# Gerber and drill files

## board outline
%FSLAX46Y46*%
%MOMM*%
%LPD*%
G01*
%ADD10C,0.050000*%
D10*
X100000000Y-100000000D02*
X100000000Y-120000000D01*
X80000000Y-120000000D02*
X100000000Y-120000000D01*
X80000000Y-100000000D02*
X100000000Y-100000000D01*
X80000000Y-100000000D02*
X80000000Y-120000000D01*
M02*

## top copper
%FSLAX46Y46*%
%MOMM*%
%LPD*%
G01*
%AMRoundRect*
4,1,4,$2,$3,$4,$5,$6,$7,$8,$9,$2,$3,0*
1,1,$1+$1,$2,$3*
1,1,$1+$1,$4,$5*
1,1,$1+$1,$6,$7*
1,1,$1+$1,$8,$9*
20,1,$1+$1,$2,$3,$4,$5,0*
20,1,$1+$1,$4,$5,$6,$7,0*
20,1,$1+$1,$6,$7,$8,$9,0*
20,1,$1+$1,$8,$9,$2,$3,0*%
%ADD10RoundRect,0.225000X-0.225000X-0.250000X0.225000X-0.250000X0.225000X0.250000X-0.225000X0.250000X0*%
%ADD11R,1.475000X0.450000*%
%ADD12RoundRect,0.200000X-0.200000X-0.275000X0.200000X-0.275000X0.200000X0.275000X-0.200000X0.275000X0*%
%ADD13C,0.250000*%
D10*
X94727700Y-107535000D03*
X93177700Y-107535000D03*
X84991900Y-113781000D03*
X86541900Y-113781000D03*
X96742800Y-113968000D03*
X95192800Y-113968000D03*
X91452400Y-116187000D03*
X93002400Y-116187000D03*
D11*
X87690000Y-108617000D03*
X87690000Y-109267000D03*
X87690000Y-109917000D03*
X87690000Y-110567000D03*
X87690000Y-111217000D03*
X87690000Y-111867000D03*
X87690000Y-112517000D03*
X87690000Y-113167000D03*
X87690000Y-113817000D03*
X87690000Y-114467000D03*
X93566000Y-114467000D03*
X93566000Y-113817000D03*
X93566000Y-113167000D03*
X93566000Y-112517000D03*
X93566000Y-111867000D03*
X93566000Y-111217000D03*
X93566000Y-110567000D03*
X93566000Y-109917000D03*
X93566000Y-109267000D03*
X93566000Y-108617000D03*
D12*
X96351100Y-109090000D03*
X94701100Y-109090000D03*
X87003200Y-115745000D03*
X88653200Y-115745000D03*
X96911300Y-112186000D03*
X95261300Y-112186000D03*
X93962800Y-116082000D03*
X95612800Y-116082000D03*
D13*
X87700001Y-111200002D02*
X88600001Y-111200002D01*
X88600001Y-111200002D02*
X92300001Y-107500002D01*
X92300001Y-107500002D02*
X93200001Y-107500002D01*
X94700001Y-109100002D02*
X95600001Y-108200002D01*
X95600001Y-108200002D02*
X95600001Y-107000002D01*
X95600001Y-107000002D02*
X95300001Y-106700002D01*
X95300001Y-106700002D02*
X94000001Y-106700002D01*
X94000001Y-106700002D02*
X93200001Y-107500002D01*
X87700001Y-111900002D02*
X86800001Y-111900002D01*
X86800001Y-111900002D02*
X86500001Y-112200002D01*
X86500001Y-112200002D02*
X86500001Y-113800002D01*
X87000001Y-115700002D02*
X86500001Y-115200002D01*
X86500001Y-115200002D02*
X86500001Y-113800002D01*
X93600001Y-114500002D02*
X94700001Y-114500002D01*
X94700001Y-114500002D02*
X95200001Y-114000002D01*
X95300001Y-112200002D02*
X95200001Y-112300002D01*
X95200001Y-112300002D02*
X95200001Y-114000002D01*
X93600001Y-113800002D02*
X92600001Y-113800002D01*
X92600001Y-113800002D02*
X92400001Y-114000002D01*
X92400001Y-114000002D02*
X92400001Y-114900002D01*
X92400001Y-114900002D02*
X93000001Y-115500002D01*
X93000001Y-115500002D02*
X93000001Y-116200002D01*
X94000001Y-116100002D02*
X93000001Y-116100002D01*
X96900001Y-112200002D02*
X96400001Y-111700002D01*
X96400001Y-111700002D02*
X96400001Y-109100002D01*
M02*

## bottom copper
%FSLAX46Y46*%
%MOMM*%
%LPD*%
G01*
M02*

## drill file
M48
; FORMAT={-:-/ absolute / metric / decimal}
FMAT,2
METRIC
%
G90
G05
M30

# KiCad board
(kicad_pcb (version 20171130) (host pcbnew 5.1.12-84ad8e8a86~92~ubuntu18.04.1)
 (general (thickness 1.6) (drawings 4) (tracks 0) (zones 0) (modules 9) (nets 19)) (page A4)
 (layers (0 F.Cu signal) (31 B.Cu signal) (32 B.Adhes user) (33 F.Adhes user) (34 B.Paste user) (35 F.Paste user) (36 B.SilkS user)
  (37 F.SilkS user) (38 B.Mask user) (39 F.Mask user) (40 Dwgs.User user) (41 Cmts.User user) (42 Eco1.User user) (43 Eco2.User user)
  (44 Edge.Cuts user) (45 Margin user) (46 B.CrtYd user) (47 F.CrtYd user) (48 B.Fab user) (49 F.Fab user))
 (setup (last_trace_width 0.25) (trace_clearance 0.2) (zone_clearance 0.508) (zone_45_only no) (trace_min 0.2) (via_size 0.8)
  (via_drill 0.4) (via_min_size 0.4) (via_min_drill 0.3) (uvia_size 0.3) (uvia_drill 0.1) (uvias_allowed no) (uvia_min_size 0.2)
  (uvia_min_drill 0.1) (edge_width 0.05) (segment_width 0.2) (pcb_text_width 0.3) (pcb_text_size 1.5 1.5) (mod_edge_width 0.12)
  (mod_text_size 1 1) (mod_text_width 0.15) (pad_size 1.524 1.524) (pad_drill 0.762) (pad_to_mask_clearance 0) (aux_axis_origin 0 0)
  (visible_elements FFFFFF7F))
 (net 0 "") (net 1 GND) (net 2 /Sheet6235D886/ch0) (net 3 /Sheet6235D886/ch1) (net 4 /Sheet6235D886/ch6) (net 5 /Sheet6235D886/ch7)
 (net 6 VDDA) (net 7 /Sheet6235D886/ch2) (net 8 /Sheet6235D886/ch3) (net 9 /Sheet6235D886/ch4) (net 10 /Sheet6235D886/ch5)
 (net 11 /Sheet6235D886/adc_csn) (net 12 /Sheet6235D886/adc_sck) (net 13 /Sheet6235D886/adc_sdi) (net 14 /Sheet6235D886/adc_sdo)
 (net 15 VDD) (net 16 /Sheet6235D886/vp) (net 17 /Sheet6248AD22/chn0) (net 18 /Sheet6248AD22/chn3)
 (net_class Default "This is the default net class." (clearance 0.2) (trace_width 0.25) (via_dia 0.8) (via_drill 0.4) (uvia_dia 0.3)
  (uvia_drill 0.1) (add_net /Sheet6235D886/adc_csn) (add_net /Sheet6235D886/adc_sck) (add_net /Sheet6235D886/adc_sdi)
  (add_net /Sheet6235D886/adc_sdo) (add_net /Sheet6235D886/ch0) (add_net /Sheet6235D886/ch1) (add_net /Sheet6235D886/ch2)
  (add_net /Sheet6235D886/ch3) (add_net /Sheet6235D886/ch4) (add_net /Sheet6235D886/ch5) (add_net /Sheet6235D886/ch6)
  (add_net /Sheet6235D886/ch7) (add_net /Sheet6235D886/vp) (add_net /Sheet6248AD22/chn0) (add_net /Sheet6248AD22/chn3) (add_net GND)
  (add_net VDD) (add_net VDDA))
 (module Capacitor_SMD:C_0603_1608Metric (layer F.Cu) (at 93.952700 107.535000)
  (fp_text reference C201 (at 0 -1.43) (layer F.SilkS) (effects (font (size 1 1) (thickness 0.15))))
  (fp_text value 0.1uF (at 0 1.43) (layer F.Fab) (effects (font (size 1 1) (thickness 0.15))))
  (pad 2 smd roundrect (at 0.775 0) (size 0.9 0.95) (layers F.Cu F.Mask F.Paste) (roundrect_rratio 0.25) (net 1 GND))
  (pad 1 smd roundrect (at -0.775 0) (size 0.9 0.95) (layers F.Cu F.Mask F.Paste) (roundrect_rratio 0.25) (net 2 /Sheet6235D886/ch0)))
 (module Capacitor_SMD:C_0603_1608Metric (layer F.Cu) (at 85.766900 113.781000)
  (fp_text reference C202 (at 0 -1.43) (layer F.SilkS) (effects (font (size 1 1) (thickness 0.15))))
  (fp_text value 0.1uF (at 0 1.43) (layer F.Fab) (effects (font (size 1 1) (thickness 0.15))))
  (pad 1 smd roundrect (at -0.775 0) (size 0.9 0.95) (layers F.Cu F.Mask F.Paste) (roundrect_rratio 0.25) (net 1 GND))
  (pad 2 smd roundrect (at 0.775 0) (size 0.9 0.95) (layers F.Cu F.Mask F.Paste) (roundrect_rratio 0.25) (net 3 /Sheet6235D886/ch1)))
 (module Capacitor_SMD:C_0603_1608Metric (layer F.Cu) (at 95.967800 113.968000)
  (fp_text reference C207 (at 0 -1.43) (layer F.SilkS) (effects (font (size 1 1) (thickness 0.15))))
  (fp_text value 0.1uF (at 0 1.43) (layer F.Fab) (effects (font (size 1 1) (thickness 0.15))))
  (pad 2 smd roundrect (at 0.775 0) (size 0.9 0.95) (layers F.Cu F.Mask F.Paste) (roundrect_rratio 0.25) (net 1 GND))
  (pad 1 smd roundrect (at -0.775 0) (size 0.9 0.95) (layers F.Cu F.Mask F.Paste) (roundrect_rratio 0.25) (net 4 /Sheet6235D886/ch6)))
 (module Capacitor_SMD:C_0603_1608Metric (layer F.Cu) (at 92.227400 116.187000)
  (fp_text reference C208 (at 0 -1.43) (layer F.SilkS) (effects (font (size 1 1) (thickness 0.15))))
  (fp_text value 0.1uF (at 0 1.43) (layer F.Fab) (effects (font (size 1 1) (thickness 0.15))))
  (pad 1 smd roundrect (at -0.775 0) (size 0.9 0.95) (layers F.Cu F.Mask F.Paste) (roundrect_rratio 0.25) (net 1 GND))
  (pad 2 smd roundrect (at 0.775 0) (size 0.9 0.95) (layers F.Cu F.Mask F.Paste) (roundrect_rratio 0.25) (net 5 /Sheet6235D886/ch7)))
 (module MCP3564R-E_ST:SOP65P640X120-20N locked (layer F.Cu) (at 90.628000 111.542000)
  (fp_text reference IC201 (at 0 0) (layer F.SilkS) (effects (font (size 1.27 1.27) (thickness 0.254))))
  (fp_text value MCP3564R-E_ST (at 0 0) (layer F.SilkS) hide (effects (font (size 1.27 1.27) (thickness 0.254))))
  (pad 1 smd rect (at -2.938 -2.925 90.000000) (size 0.45 1.475) (layers F.Cu F.Mask F.Paste) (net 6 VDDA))
  (pad 2 smd rect (at -2.938 -2.275 90.000000) (size 0.45 1.475) (layers F.Cu F.Mask F.Paste) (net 1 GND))
  (pad 3 smd rect (at -2.938 -1.625 90.000000) (size 0.45 1.475) (layers F.Cu F.Mask F.Paste) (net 1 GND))
  (pad 4 smd rect (at -2.938 -0.975 90.000000) (size 0.45 1.475) (layers F.Cu F.Mask F.Paste))
  (pad 5 smd rect (at -2.938 -0.325 90.000000) (size 0.45 1.475) (layers F.Cu F.Mask F.Paste) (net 2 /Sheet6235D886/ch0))
  (pad 6 smd rect (at -2.938 0.325 90.000000) (size 0.45 1.475) (layers F.Cu F.Mask F.Paste) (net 3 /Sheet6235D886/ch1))
  (pad 7 smd rect (at -2.938 0.975 90.000000) (size 0.45 1.475) (layers F.Cu F.Mask F.Paste) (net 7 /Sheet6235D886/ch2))
  (pad 8 smd rect (at -2.938 1.625 90.000000) (size 0.45 1.475) (layers F.Cu F.Mask F.Paste) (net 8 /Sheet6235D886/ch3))
  (pad 9 smd rect (at -2.938 2.275 90.000000) (size 0.45 1.475) (layers F.Cu F.Mask F.Paste) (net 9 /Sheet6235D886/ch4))
  (pad 10 smd rect (at -2.938 2.925 90.000000) (size 0.45 1.475) (layers F.Cu F.Mask F.Paste) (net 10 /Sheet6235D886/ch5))
  (pad 11 smd rect (at 2.938 2.925 90.000000) (size 0.45 1.475) (layers F.Cu F.Mask F.Paste) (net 4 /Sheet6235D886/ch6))
  (pad 12 smd rect (at 2.938 2.275 90.000000) (size 0.45 1.475) (layers F.Cu F.Mask F.Paste) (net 5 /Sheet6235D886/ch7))
  (pad 13 smd rect (at 2.938 1.625 90.000000) (size 0.45 1.475) (layers F.Cu F.Mask F.Paste) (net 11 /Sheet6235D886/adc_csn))
  (pad 14 smd rect (at 2.938 0.975 90.000000) (size 0.45 1.475) (layers F.Cu F.Mask F.Paste) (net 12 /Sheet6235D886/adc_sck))
  (pad 15 smd rect (at 2.938 0.325 90.000000) (size 0.45 1.475) (layers F.Cu F.Mask F.Paste) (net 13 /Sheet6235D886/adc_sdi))
  (pad 16 smd rect (at 2.938 -0.325 90.000000) (size 0.45 1.475) (layers F.Cu F.Mask F.Paste) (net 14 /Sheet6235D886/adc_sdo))
  (pad 17 smd rect (at 2.938 -0.975 90.000000) (size 0.45 1.475) (layers F.Cu F.Mask F.Paste))
  (pad 18 smd rect (at 2.938 -1.625 90.000000) (size 0.45 1.475) (layers F.Cu F.Mask F.Paste))
  (pad 19 smd rect (at 2.938 -2.275 90.000000) (size 0.45 1.475) (layers F.Cu F.Mask F.Paste) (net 1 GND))
  (pad 20 smd rect (at 2.938 -2.925 90.000000) (size 0.45 1.475) (layers F.Cu F.Mask F.Paste) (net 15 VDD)))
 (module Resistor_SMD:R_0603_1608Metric (layer F.Cu) (at 95.526100 109.090000)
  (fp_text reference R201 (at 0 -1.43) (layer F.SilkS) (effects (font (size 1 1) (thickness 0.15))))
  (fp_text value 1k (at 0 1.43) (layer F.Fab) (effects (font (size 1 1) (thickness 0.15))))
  (pad 2 smd roundrect (at 0.825 0) (size 0.8 0.95) (layers F.Cu F.Mask F.Paste) (roundrect_rratio 0.25) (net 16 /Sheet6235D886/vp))
  (pad 1 smd roundrect (at -0.825 0) (size 0.8 0.95) (layers F.Cu F.Mask F.Paste) (roundrect_rratio 0.25) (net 2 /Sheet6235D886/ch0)))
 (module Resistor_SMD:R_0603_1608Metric (layer F.Cu) (at 87.828200 115.745000)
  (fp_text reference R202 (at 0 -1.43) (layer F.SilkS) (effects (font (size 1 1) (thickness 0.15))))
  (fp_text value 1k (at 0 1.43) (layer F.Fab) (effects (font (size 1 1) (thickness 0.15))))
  (pad 1 smd roundrect (at -0.825 0) (size 0.8 0.95) (layers F.Cu F.Mask F.Paste) (roundrect_rratio 0.25) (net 3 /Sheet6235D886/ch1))
  (pad 2 smd roundrect (at 0.825 0) (size 0.8 0.95) (layers F.Cu F.Mask F.Paste) (roundrect_rratio 0.25) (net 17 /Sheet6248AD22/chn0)))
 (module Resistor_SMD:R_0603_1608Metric (layer F.Cu) (at 96.086300 112.186000)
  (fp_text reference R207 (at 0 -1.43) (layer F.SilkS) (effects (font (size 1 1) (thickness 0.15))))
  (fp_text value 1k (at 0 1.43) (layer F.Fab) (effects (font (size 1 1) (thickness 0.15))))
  (pad 2 smd roundrect (at 0.825 0) (size 0.8 0.95) (layers F.Cu F.Mask F.Paste) (roundrect_rratio 0.25) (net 16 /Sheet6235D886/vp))
  (pad 1 smd roundrect (at -0.825 0) (size 0.8 0.95) (layers F.Cu F.Mask F.Paste) (roundrect_rratio 0.25) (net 4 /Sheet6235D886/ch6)))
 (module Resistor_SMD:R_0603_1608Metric (layer F.Cu) (at 94.787800 116.082000)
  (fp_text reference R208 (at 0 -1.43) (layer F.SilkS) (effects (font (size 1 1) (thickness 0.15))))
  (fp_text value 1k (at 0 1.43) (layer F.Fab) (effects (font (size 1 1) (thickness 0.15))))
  (pad 1 smd roundrect (at -0.825 0) (size 0.8 0.95) (layers F.Cu F.Mask F.Paste) (roundrect_rratio 0.25) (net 5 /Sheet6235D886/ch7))
  (pad 2 smd roundrect (at 0.825 0) (size 0.8 0.95) (layers F.Cu F.Mask F.Paste) (roundrect_rratio 0.25) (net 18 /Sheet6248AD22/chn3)))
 (gr_line (start 100 100) (end 100 120) (layer Edge.Cuts) (width 0.05))
 (gr_line (start 80 120) (end 100 120) (layer Edge.Cuts) (width 0.05))
 (gr_line (start 80 100) (end 100 100) (layer Edge.Cuts) (width 0.05))
 (gr_line (start 80 100) (end 80 120) (layer Edge.Cuts) (width 0.05))
 (segment (start 87.700001 111.200002) (end 88.600001 111.200002) (width 0.250000) (layer F.Cu) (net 2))
 (segment (start 88.600001 111.200002) (end 92.300001 107.500002) (width 0.250000) (layer F.Cu) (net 2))
 (segment (start 92.300001 107.500002) (end 93.200001 107.500002) (width 0.250000) (layer F.Cu) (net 2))
 (segment (start 94.700001 109.100002) (end 95.600001 108.200002) (width 0.250000) (layer F.Cu) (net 2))
 (segment (start 95.600001 108.200002) (end 95.600001 107.000002) (width 0.250000) (layer F.Cu) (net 2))
 (segment (start 95.600001 107.000002) (end 95.300001 106.700002) (width 0.250000) (layer F.Cu) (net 2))
 (segment (start 95.300001 106.700002) (end 94.000001 106.700002) (width 0.250000) (layer F.Cu) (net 2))
 (segment (start 94.000001 106.700002) (end 93.200001 107.500002) (width 0.250000) (layer F.Cu) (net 2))
 (segment (start 87.700001 111.900002) (end 86.800001 111.900002) (width 0.250000) (layer F.Cu) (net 3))
 (segment (start 86.800001 111.900002) (end 86.500001 112.200002) (width 0.250000) (layer F.Cu) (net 3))
 (segment (start 86.500001 112.200002) (end 86.500001 113.800002) (width 0.250000) (layer F.Cu) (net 3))
 (segment (start 87.000001 115.700002) (end 86.500001 115.200002) (width 0.250000) (layer F.Cu) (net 3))
 (segment (start 86.500001 115.200002) (end 86.500001 113.800002) (width 0.250000) (layer F.Cu) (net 3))
 (segment (start 93.600001 114.500002) (end 94.700001 114.500002) (width 0.250000) (layer F.Cu) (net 4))
 (segment (start 94.700001 114.500002) (end 95.200001 114.000002) (width 0.250000) (layer F.Cu) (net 4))
 (segment (start 95.300001 112.200002) (end 95.200001 112.300002) (width 0.250000) (layer F.Cu) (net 4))
 (segment (start 95.200001 112.300002) (end 95.200001 114.000002) (width 0.250000) (layer F.Cu) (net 4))
 (segment (start 93.600001 113.800002) (end 92.600001 113.800002) (width 0.250000) (layer F.Cu) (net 5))
 (segment (start 92.600001 113.800002) (end 92.400001 114.000002) (width 0.250000) (layer F.Cu) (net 5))
 (segment (start 92.400001 114.000002) (end 92.400001 114.900002) (width 0.250000) (layer F.Cu) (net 5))
 (segment (start 92.400001 114.900002) (end 93.000001 115.500002) (width 0.250000) (layer F.Cu) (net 5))
 (segment (start 93.000001 115.500002) (end 93.000001 116.200002) (width 0.250000) (layer F.Cu) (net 5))
 (segment (start 94.000001 116.100002) (end 93.000001 116.100002) (width 0.250000) (layer F.Cu) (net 5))
 (segment (start 96.900001 112.200002) (end 96.400001 111.700002) (width 0.250000) (layer F.Cu) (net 16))
 (segment (start 96.400001 111.700002) (end 96.400001 109.100002) (width 0.250000) (layer F.Cu) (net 16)))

